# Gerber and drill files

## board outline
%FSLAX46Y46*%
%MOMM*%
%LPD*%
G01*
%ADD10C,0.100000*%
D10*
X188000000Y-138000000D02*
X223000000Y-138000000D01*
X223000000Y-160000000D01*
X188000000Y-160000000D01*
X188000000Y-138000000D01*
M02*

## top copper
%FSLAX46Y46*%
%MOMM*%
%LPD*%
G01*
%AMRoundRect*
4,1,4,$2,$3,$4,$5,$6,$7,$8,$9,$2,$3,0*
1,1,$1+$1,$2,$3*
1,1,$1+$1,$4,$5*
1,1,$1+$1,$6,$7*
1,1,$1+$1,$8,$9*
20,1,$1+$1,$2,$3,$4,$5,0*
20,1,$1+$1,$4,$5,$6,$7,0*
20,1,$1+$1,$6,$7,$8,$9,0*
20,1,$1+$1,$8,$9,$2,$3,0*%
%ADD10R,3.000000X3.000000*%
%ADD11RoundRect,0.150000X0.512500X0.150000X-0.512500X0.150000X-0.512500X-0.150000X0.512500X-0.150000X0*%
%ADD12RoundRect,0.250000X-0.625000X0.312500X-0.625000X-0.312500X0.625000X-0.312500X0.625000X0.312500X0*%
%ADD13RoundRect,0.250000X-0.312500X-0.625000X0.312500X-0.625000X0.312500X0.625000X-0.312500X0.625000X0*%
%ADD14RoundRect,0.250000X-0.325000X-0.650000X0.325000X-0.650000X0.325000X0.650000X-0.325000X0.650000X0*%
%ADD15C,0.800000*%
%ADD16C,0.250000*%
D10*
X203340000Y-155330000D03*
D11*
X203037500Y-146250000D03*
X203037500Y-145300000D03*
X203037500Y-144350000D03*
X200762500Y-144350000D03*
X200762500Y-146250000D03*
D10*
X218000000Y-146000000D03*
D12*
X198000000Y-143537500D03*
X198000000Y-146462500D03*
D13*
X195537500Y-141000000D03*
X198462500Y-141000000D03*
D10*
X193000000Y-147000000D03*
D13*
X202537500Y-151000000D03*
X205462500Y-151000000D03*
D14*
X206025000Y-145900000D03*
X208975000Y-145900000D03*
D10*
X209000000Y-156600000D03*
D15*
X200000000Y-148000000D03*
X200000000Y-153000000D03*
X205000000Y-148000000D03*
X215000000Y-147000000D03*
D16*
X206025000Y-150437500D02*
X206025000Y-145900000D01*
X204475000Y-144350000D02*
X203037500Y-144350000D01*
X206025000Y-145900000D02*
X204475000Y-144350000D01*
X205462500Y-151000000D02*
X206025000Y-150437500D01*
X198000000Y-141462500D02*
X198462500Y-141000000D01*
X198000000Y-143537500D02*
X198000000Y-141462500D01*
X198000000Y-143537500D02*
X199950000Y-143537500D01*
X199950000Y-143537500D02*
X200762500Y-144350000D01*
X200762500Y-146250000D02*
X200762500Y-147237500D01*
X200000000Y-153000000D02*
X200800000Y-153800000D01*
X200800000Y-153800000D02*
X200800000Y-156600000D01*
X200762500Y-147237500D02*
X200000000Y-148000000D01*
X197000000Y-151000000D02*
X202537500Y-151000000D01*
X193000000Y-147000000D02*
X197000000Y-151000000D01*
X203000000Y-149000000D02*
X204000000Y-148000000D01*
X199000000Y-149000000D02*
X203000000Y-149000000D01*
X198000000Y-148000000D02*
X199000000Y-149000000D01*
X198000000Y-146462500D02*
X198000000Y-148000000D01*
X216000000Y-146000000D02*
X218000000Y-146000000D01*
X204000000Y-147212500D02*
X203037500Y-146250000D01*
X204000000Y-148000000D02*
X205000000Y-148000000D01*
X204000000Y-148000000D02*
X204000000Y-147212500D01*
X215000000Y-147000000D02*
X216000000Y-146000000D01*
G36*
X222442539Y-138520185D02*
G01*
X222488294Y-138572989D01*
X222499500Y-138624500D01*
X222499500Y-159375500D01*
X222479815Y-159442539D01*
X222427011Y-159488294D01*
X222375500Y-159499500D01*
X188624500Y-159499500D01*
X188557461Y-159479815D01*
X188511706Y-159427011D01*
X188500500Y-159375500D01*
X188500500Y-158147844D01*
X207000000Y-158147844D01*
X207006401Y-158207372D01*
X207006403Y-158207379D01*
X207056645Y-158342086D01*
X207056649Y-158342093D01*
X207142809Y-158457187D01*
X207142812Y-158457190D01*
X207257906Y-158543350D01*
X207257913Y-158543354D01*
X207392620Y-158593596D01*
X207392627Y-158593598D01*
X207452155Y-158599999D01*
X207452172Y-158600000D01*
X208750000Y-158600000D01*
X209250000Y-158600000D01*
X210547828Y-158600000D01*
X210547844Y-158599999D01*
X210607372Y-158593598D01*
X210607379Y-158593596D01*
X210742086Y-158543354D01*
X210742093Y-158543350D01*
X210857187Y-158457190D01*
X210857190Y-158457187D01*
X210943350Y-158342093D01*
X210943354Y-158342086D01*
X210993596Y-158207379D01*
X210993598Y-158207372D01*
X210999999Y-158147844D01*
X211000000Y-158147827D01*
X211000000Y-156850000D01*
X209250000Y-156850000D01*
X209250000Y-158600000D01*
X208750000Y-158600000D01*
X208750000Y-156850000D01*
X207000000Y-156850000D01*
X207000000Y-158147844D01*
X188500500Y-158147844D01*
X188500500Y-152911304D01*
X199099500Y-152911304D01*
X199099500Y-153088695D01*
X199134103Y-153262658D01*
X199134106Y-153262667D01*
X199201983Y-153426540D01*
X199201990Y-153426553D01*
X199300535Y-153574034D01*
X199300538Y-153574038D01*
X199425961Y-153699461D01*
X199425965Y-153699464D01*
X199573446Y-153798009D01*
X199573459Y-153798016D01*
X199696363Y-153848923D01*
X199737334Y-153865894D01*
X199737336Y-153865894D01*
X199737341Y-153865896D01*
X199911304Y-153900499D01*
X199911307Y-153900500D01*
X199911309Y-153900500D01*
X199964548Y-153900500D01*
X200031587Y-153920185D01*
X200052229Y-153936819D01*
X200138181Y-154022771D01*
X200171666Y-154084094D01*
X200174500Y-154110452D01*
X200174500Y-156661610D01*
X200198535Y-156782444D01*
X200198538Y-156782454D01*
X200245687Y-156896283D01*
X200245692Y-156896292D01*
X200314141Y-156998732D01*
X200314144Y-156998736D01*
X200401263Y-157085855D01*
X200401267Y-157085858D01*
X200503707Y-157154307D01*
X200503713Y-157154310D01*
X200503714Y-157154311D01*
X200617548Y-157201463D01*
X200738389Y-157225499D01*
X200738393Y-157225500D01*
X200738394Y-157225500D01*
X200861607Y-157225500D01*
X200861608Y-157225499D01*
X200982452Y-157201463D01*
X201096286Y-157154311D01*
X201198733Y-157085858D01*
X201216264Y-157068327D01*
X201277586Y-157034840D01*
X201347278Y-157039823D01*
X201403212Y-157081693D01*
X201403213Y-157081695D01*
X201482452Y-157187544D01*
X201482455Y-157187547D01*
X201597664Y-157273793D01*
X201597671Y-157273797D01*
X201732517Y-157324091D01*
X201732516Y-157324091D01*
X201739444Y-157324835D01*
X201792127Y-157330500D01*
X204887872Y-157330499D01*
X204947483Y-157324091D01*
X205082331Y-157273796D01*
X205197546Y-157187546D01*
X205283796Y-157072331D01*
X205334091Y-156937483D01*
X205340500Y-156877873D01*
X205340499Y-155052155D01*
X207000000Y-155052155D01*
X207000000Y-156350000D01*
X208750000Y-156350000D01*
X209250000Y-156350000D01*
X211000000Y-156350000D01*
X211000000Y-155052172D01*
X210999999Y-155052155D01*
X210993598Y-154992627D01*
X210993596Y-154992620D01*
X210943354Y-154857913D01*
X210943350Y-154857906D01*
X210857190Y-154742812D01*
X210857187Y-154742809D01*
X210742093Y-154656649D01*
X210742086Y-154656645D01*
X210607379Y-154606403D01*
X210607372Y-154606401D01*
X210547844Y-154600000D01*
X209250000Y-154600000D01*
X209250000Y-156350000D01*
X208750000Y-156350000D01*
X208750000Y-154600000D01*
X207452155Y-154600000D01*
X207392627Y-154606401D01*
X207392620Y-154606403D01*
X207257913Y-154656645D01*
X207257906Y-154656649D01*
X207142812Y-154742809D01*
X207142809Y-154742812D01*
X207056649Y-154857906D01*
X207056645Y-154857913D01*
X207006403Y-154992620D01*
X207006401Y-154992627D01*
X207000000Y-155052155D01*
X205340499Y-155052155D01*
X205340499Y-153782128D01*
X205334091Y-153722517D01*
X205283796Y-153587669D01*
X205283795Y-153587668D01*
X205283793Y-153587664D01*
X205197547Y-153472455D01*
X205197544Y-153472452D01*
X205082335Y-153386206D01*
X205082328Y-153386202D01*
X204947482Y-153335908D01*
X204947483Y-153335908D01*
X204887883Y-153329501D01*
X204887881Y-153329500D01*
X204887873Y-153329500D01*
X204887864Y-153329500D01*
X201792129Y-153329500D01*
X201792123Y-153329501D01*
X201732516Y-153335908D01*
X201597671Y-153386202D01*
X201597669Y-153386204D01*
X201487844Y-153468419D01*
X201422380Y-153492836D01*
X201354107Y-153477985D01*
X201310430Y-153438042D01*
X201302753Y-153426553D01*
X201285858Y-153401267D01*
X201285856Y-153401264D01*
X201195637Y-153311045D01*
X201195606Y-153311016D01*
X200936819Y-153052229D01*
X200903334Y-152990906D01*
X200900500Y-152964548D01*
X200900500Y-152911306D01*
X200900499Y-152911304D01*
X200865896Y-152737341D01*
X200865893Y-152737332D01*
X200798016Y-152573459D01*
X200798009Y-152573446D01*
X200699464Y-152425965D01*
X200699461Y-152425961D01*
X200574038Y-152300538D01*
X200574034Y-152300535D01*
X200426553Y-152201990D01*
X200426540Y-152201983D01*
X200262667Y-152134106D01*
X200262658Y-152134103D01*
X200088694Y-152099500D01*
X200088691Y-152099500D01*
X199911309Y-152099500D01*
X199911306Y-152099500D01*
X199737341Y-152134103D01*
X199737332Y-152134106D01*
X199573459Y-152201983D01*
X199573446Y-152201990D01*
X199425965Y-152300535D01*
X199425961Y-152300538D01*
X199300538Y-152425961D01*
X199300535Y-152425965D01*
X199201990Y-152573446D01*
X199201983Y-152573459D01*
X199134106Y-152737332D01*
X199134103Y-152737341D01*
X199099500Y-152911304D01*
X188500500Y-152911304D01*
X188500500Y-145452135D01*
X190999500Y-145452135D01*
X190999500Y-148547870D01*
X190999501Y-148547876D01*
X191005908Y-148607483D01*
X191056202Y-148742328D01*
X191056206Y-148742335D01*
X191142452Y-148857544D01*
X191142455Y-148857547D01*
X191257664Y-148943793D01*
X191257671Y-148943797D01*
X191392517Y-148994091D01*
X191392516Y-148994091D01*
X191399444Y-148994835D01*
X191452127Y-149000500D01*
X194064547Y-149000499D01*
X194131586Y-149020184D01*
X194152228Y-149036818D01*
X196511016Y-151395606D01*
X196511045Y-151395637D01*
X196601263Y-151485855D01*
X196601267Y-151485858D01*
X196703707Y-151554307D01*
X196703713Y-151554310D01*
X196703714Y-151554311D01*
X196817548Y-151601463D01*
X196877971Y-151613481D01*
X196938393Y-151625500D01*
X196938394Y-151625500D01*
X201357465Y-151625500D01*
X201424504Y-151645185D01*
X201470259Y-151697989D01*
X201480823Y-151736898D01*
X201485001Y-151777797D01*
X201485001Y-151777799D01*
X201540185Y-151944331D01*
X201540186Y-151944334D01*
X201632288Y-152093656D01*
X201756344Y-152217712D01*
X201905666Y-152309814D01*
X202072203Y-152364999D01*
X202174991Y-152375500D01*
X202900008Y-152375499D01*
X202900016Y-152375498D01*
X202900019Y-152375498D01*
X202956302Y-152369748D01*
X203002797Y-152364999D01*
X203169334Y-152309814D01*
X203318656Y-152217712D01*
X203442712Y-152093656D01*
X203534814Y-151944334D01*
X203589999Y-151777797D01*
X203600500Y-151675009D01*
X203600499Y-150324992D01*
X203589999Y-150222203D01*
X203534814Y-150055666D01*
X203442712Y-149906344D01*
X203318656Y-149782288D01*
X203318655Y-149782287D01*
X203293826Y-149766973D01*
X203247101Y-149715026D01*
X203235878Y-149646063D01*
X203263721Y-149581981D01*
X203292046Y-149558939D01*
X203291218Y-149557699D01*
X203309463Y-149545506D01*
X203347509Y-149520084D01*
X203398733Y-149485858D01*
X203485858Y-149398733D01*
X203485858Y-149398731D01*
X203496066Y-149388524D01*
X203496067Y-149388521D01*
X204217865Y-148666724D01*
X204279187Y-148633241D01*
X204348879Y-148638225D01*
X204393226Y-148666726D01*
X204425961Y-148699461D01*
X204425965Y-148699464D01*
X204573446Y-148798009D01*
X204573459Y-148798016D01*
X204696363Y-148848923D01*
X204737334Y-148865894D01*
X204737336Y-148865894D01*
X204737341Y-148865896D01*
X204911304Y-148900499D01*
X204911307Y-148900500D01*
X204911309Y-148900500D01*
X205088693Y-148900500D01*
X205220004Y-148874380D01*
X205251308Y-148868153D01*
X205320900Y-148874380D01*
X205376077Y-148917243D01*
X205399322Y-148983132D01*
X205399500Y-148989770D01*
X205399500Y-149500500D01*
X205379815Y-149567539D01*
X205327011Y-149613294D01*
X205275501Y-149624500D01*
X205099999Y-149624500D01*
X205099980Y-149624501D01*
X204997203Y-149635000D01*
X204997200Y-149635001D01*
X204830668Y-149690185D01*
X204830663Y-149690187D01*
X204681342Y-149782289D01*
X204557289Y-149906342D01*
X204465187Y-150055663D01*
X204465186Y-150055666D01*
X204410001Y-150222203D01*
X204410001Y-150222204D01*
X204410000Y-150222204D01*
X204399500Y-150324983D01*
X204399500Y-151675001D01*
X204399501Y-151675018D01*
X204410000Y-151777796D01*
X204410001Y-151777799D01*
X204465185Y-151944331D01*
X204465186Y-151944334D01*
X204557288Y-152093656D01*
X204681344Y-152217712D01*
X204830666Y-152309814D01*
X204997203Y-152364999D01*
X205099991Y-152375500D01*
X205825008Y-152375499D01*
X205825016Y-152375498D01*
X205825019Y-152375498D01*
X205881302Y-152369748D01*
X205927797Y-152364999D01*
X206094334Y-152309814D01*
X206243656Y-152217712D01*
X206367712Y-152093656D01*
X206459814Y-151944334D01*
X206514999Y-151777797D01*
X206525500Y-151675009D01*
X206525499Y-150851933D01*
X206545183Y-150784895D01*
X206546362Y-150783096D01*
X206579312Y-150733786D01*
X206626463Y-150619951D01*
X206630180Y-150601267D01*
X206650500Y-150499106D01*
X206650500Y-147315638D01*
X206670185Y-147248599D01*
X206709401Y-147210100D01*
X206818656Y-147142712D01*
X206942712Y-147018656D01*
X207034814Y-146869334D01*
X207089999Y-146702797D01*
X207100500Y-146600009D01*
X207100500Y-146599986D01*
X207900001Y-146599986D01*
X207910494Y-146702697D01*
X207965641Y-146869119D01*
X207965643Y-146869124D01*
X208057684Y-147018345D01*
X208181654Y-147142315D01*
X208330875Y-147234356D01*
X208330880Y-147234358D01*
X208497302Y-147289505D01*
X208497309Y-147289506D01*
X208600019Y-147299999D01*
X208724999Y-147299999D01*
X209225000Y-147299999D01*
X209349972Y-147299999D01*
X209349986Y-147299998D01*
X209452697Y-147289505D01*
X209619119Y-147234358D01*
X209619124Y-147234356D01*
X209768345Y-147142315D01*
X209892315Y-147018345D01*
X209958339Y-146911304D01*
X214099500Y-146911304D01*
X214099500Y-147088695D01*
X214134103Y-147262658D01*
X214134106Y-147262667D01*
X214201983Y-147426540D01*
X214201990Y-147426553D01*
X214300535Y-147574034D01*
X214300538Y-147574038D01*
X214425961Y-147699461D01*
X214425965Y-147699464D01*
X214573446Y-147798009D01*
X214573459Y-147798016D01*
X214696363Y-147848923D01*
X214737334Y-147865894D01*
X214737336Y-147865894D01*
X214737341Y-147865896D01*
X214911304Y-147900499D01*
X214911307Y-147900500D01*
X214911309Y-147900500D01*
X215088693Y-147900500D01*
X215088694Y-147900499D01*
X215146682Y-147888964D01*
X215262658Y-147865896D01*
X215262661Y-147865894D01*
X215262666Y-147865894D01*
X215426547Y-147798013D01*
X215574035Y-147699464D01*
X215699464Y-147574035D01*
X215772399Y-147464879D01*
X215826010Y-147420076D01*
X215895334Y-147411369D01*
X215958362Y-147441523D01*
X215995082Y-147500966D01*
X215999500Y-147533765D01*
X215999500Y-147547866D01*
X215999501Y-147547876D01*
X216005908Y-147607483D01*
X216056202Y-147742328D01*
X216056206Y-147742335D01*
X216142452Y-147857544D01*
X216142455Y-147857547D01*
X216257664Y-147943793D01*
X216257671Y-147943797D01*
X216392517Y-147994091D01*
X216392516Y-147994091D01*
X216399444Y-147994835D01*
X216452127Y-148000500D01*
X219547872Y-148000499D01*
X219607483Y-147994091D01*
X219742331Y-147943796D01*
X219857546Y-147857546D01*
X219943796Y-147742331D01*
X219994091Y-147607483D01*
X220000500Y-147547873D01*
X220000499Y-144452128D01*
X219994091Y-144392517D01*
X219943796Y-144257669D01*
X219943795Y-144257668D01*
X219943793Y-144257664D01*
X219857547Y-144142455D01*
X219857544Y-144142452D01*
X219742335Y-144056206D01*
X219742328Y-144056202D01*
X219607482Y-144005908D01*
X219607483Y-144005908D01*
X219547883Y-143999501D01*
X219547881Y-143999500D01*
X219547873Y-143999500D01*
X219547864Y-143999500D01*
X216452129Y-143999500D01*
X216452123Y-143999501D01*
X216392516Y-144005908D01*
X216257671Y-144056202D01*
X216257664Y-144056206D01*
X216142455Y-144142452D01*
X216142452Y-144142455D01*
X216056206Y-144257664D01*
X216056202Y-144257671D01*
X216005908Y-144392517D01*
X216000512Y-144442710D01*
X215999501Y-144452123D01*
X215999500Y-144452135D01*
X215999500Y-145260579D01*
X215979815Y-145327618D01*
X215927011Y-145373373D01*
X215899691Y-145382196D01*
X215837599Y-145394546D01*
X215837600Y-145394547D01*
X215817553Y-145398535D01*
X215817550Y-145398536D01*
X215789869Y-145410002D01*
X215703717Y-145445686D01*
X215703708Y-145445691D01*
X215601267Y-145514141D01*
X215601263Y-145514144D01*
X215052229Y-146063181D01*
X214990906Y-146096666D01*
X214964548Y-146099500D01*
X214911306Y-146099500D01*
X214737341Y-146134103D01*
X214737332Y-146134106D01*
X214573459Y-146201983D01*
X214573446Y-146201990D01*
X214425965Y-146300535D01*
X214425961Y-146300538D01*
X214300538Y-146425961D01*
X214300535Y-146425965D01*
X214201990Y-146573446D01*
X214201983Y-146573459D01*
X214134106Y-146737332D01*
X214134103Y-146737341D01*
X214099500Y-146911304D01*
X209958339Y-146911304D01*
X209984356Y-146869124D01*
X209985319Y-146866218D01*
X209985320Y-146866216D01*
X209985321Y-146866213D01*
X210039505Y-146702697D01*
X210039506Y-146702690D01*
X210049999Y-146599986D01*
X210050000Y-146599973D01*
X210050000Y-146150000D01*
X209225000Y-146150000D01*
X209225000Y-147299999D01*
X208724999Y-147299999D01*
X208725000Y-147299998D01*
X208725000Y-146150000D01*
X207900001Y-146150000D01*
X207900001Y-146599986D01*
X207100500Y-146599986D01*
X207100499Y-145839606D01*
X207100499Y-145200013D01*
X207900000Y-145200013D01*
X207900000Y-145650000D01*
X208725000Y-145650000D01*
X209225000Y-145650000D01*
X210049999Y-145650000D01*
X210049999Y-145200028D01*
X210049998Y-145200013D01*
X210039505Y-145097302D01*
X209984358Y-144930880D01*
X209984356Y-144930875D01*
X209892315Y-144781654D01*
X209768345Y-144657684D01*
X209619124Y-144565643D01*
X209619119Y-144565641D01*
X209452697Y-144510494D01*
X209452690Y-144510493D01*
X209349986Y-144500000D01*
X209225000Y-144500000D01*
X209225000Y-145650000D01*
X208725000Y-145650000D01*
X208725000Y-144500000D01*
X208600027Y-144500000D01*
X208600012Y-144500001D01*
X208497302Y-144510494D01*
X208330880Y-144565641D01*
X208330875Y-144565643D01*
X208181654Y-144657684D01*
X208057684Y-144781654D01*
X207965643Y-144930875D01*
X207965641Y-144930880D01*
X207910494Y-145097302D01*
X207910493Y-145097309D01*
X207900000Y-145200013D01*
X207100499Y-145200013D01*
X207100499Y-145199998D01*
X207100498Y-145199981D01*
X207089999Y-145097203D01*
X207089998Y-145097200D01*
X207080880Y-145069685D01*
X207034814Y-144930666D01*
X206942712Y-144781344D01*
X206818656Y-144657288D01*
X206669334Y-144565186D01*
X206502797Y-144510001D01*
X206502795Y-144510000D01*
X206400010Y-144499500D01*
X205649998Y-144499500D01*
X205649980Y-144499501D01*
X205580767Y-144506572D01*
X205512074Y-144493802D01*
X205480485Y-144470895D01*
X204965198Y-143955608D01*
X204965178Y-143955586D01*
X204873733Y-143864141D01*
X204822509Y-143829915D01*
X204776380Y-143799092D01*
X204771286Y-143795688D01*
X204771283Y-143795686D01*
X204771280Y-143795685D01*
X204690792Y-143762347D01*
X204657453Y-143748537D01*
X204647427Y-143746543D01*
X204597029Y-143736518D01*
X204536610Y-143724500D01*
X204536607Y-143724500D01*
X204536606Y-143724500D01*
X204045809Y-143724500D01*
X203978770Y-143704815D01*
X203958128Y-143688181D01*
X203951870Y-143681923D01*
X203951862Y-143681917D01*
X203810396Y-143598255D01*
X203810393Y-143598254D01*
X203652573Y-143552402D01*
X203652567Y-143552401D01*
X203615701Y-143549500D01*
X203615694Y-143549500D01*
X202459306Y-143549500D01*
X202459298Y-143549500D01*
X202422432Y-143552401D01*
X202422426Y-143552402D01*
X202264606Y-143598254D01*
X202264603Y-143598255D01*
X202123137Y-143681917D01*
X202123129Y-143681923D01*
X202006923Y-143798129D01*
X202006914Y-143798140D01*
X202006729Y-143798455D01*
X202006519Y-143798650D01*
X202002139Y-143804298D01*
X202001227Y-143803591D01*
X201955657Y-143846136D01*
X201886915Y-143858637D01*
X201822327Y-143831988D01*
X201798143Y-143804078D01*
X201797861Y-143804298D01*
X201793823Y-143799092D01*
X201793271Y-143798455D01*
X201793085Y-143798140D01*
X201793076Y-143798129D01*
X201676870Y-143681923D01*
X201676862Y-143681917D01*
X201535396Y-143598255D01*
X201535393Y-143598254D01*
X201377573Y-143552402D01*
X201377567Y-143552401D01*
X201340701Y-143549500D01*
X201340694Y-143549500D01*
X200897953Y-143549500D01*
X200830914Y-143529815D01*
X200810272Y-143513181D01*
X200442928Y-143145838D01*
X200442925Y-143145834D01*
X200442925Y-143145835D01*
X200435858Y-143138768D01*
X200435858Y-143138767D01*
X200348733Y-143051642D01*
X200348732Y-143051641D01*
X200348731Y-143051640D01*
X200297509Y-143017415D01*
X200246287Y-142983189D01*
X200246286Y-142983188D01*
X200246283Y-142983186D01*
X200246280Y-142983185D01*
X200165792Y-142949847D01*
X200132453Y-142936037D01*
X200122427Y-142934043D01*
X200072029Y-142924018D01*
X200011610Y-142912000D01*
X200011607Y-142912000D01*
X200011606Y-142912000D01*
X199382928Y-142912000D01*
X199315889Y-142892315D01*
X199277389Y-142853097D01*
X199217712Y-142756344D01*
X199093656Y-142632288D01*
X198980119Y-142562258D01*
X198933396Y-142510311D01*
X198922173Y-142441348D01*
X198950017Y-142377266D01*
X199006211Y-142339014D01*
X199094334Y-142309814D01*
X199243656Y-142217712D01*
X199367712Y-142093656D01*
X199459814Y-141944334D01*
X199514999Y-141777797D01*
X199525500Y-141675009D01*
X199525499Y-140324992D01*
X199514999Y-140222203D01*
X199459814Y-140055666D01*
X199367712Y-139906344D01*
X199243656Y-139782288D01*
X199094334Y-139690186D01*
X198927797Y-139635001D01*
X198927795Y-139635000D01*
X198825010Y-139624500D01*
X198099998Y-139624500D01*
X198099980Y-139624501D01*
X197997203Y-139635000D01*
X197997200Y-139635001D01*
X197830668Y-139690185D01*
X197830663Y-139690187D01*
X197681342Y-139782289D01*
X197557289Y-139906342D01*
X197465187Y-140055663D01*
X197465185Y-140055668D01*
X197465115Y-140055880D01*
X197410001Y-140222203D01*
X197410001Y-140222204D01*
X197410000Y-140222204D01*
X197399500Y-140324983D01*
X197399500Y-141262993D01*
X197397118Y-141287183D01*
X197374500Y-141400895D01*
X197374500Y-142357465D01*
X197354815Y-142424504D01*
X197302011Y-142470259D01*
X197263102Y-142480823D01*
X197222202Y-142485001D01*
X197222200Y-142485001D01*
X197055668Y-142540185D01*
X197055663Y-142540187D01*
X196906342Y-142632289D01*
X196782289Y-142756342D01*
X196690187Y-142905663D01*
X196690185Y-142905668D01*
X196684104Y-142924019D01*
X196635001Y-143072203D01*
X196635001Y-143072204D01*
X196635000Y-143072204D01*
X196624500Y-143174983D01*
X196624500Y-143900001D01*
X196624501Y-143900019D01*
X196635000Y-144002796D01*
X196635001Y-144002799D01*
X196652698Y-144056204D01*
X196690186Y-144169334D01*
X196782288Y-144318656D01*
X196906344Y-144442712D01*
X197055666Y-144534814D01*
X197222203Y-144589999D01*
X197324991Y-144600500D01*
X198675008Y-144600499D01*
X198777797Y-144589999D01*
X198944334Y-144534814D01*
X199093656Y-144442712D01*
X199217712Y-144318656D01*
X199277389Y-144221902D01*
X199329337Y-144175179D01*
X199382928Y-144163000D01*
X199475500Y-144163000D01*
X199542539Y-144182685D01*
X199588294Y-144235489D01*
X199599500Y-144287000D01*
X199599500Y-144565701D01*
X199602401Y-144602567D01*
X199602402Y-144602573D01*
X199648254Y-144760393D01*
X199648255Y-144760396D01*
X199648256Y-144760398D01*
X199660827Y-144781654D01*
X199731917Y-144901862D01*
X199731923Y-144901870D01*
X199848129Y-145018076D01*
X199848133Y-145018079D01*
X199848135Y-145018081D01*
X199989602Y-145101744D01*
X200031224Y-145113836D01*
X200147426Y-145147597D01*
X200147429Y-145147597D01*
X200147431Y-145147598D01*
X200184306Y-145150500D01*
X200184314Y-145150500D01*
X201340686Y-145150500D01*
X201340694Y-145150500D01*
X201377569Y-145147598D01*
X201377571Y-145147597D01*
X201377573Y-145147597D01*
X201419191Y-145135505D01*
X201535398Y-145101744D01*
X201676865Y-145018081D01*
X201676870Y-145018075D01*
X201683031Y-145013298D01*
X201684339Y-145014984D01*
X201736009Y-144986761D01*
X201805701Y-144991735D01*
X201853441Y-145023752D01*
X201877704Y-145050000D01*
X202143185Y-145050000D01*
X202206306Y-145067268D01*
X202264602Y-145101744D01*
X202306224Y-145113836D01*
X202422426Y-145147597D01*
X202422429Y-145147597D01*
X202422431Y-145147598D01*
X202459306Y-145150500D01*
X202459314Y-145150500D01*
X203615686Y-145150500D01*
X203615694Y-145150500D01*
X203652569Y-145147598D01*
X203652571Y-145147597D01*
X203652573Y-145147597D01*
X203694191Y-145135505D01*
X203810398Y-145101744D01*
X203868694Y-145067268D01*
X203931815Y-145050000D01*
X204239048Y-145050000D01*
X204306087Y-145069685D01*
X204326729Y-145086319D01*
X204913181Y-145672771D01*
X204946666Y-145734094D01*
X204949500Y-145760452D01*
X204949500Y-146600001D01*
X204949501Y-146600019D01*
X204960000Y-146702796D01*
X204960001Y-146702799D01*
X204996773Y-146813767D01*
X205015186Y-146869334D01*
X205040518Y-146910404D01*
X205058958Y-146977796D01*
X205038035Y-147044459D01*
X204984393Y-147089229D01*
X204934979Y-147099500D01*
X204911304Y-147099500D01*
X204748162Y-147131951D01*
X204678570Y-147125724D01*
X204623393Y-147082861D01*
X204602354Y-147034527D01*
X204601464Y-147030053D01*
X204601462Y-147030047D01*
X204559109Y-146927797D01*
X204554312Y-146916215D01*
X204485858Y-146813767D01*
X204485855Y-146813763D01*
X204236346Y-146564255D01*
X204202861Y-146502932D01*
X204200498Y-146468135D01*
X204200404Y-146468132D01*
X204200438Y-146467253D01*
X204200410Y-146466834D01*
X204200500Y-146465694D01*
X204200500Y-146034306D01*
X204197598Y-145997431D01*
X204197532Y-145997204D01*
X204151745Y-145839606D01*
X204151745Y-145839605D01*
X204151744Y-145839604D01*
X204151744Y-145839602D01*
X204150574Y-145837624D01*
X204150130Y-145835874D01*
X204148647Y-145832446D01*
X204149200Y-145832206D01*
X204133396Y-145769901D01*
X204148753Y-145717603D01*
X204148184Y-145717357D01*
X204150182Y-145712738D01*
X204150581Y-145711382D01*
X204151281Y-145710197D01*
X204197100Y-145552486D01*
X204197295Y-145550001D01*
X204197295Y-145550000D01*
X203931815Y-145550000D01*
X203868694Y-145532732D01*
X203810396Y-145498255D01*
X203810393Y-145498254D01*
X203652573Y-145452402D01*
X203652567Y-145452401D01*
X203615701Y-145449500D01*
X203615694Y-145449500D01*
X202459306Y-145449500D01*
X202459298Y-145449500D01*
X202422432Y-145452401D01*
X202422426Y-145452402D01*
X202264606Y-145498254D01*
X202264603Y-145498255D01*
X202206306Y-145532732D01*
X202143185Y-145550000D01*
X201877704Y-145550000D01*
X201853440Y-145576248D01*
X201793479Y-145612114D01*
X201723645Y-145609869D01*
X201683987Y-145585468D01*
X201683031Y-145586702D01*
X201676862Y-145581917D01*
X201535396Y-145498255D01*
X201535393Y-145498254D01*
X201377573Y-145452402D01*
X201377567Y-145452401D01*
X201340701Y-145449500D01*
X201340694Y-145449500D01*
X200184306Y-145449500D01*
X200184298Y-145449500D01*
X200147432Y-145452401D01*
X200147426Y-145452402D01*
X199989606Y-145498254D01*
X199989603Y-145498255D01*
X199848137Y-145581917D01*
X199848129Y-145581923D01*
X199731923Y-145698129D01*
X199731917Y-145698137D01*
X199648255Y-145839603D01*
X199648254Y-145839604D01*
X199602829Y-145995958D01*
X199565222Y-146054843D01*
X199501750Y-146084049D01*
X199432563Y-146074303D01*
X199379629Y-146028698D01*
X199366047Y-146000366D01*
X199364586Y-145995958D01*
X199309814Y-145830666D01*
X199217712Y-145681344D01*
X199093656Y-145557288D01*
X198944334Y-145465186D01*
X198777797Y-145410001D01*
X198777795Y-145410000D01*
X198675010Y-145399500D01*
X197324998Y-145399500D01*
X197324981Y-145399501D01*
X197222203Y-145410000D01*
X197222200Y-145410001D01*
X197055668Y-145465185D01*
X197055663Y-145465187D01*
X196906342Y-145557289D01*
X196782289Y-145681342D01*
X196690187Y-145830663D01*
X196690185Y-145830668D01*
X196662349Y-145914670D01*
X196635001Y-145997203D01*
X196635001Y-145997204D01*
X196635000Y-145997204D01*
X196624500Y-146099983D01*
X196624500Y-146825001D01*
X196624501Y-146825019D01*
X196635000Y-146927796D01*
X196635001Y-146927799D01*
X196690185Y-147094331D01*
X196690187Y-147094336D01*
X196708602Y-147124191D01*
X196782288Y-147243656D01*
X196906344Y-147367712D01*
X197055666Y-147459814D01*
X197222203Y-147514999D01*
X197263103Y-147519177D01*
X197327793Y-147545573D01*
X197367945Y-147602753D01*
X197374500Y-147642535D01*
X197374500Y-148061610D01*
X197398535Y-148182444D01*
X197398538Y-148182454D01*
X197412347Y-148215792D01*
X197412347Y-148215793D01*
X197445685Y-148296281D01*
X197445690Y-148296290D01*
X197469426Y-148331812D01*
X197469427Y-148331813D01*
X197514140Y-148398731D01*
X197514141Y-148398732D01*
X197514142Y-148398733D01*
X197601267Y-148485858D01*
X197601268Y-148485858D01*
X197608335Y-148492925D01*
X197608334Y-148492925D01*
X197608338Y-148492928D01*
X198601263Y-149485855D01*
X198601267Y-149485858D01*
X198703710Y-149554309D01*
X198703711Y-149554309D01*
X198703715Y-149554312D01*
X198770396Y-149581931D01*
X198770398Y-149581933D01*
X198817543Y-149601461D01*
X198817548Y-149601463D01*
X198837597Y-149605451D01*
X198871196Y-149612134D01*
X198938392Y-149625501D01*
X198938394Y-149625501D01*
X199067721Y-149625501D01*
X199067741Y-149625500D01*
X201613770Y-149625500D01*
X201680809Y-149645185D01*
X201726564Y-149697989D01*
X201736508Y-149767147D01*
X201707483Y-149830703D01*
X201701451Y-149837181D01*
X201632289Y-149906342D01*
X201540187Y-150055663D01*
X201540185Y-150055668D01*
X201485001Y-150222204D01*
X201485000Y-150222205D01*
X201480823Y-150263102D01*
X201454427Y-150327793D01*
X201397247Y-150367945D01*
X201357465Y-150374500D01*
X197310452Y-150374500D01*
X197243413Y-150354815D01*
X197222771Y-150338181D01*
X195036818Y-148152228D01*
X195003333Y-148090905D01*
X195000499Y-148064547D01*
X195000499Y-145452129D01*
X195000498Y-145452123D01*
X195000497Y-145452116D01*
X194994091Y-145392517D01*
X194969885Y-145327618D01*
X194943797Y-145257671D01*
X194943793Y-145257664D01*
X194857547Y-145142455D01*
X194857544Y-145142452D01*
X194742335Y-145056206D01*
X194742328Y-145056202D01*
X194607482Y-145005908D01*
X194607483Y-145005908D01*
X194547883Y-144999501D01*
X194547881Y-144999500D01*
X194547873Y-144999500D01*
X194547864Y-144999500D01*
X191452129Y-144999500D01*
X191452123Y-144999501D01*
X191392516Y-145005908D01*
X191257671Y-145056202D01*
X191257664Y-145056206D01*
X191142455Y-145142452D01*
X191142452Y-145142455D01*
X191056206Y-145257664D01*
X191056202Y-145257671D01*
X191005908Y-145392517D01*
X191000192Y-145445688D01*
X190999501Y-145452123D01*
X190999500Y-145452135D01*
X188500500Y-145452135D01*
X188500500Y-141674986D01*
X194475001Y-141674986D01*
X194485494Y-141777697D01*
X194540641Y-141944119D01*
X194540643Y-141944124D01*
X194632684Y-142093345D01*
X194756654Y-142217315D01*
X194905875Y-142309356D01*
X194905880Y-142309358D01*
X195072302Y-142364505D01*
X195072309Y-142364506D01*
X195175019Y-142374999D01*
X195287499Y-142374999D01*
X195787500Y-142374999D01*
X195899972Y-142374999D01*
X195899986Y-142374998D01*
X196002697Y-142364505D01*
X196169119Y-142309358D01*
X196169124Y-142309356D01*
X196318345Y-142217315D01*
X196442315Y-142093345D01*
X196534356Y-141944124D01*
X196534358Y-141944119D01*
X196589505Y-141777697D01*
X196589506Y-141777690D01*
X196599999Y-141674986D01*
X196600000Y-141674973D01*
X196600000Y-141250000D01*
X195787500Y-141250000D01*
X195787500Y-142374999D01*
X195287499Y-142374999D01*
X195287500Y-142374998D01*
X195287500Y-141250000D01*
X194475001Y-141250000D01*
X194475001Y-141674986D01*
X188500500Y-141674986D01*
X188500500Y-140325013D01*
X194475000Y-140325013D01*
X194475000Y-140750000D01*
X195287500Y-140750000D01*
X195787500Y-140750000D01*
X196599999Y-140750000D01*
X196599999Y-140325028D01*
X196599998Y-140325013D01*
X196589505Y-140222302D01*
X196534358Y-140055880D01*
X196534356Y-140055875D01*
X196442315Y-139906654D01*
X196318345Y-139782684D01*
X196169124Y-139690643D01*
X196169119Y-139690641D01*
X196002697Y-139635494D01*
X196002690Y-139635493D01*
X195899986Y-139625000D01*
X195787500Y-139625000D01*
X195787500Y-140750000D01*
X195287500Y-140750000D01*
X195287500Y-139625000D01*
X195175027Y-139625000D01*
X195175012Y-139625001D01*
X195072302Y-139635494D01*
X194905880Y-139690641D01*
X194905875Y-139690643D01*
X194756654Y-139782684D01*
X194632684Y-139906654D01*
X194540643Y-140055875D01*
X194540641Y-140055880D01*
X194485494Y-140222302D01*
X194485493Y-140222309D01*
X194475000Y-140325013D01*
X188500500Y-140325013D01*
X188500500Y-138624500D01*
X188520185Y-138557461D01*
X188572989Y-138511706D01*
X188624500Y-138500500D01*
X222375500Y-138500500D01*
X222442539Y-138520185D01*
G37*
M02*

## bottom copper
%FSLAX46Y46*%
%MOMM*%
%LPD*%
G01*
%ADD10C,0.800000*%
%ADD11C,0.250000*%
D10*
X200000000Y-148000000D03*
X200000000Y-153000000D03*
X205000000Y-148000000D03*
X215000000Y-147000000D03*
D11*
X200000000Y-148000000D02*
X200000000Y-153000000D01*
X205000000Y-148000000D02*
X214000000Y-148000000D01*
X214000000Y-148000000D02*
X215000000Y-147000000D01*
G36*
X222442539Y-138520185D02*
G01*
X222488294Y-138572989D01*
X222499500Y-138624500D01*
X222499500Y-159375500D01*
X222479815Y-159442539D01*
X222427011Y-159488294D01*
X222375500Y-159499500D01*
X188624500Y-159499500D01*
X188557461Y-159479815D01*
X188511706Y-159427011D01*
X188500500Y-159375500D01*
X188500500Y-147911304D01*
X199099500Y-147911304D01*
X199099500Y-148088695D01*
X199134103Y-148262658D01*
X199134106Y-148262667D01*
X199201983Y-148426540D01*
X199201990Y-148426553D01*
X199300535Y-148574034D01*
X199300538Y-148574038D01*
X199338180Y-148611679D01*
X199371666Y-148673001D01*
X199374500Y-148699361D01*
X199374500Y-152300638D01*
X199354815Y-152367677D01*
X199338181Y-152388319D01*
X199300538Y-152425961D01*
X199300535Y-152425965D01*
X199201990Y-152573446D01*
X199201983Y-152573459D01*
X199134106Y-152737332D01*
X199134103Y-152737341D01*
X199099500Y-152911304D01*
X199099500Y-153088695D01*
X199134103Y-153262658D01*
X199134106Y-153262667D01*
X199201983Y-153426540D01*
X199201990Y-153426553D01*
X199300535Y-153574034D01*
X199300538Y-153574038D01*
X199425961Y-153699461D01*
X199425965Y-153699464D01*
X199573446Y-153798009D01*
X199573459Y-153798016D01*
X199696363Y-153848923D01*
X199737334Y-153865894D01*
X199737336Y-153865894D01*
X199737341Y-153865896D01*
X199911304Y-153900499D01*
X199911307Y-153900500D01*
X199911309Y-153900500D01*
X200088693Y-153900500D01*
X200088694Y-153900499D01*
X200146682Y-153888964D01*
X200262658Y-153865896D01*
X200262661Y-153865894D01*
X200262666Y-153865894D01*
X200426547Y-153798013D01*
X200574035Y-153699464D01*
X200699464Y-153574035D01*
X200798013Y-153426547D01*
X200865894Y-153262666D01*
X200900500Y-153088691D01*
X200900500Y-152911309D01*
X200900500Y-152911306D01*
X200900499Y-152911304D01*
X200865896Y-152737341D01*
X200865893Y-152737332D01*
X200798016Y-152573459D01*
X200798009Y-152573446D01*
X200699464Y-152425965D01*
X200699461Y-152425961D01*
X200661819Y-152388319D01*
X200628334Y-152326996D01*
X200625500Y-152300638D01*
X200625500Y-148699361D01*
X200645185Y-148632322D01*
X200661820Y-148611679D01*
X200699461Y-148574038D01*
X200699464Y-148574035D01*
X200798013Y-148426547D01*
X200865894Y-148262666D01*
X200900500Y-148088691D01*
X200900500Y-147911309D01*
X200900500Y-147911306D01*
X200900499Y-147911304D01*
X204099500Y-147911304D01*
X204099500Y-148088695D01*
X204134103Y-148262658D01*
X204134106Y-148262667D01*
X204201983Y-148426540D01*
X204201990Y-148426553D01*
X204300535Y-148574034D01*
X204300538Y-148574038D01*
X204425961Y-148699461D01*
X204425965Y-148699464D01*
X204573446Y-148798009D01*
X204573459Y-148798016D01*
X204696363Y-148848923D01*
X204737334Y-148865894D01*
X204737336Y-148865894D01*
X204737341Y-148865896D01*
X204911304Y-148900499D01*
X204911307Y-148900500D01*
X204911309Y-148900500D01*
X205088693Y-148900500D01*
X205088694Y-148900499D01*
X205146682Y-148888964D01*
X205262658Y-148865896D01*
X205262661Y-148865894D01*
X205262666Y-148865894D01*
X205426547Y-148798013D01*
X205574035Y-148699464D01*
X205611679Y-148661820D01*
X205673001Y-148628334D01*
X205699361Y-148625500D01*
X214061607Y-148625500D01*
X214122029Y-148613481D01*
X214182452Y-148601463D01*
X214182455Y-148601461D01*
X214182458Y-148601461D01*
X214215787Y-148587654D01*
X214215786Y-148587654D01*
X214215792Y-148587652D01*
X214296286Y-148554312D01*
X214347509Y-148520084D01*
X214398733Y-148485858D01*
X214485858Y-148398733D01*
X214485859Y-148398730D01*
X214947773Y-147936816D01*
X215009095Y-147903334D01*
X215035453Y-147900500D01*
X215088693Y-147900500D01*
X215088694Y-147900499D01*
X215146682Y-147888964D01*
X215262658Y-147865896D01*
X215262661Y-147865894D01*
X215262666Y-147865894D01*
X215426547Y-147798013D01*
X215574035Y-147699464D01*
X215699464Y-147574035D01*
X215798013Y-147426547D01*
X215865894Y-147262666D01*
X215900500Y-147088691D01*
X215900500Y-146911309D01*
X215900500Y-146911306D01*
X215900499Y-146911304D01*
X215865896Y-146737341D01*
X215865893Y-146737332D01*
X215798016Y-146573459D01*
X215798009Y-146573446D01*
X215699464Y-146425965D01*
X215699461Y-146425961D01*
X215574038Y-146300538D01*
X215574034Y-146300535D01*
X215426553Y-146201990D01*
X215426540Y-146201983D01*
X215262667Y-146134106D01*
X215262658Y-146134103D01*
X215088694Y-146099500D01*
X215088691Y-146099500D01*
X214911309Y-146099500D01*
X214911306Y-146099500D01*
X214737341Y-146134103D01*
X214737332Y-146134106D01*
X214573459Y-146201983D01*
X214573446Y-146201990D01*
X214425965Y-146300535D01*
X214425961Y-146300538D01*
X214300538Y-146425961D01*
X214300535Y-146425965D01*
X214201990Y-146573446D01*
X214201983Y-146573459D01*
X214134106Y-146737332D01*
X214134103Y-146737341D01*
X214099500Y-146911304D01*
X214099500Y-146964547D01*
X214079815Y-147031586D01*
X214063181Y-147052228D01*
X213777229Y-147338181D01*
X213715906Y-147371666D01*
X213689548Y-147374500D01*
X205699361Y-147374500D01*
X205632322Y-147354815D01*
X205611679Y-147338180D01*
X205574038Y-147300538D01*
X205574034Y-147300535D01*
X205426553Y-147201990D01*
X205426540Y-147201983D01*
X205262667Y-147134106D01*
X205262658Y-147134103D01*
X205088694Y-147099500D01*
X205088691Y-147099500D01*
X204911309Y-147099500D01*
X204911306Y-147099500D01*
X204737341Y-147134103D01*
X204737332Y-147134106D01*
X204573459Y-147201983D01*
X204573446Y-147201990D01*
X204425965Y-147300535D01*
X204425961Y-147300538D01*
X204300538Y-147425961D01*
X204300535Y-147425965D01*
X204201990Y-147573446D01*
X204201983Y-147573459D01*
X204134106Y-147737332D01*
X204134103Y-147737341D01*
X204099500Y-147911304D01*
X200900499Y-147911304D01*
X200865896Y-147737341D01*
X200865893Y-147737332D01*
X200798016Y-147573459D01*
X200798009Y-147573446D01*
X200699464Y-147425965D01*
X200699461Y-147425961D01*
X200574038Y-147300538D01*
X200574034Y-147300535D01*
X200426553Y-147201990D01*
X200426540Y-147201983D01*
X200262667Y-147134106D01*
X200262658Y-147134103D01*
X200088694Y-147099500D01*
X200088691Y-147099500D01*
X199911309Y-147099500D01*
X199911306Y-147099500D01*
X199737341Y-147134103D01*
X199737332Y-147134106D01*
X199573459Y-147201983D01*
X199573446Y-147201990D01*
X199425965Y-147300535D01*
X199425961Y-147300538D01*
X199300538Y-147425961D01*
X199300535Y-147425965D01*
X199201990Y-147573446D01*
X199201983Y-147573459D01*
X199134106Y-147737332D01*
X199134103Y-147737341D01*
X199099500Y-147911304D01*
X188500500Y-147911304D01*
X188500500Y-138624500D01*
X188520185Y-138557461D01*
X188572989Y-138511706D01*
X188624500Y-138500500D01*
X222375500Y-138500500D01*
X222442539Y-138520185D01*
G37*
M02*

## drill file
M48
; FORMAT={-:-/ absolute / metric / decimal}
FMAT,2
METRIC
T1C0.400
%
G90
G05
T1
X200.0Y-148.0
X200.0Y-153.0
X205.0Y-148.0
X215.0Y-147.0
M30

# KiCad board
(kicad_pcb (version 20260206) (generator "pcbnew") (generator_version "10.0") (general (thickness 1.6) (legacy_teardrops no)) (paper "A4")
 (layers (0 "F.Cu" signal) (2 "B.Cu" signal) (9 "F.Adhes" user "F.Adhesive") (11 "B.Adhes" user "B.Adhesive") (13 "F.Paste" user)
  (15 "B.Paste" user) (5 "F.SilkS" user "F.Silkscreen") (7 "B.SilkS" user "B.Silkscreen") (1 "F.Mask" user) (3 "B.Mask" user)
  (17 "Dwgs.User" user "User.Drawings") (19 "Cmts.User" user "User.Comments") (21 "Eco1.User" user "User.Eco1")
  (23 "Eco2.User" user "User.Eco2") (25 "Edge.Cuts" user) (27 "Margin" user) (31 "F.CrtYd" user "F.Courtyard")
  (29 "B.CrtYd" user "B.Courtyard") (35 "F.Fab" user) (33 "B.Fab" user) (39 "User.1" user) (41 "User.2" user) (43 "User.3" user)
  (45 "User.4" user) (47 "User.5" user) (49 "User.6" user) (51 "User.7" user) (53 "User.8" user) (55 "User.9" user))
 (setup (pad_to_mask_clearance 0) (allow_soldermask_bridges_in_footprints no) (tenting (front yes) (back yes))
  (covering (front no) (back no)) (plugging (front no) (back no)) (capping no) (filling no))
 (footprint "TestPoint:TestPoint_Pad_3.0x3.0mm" (layer "F.Cu") (at 203.34 155.33)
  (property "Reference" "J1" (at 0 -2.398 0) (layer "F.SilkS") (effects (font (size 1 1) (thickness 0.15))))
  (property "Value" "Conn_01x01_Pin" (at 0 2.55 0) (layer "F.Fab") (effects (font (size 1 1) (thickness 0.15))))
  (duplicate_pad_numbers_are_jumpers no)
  (pad "1" smd rect (at 0 0) (size 3 3) (layers "F.Cu" "F.Mask") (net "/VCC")))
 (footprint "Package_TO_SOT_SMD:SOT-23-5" (layer "F.Cu") (at 201.9 145.3 180)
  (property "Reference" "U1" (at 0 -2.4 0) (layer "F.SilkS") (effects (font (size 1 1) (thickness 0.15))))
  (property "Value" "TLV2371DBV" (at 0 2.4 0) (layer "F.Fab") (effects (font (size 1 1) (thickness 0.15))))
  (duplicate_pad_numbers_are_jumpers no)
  (pad "1" smd roundrect (at -1.1375 -0.95 180) (size 1.325 0.6) (layers "F.Cu" "F.Mask" "F.Paste") (roundrect_rratio 0.25) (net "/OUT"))
  (pad "2" smd roundrect (at -1.1375 0 180) (size 1.325 0.6) (layers "F.Cu" "F.Mask" "F.Paste") (roundrect_rratio 0.25) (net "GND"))
  (pad "3" smd roundrect (at -1.1375 0.95 180) (size 1.325 0.6) (layers "F.Cu" "F.Mask" "F.Paste") (roundrect_rratio 0.25)
   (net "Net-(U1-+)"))
  (pad "4" smd roundrect (at 1.1375 0.95 180) (size 1.325 0.6) (layers "F.Cu" "F.Mask" "F.Paste") (roundrect_rratio 0.25) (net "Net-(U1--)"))
  (pad "5" smd roundrect (at 1.1375 -0.95 180) (size 1.325 0.6) (layers "F.Cu" "F.Mask" "F.Paste") (roundrect_rratio 0.25) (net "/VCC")))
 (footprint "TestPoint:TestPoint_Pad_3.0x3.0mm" (layer "F.Cu") (at 218 146)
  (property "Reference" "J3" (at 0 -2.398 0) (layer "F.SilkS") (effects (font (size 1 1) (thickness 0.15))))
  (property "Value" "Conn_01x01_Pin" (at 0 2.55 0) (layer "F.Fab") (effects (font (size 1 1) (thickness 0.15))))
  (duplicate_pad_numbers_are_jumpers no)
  (pad "1" smd rect (at 0 0) (size 3 3) (layers "F.Cu" "F.Mask") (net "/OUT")))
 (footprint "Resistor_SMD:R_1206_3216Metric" (layer "F.Cu") (at 198 145 -90)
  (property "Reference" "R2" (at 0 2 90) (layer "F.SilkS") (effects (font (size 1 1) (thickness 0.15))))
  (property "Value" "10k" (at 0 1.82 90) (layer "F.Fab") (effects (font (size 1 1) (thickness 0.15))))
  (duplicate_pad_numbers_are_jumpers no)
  (pad "1" smd roundrect (at -1.4625 0 270) (size 1.125 1.75) (layers "F.Cu" "F.Mask" "F.Paste") (roundrect_rratio 0.222222)
   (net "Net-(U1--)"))
  (pad "2" smd roundrect (at 1.4625 0 270) (size 1.125 1.75) (layers "F.Cu" "F.Mask" "F.Paste") (roundrect_rratio 0.222222) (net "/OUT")))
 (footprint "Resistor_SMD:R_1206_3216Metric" (layer "F.Cu") (at 197 141)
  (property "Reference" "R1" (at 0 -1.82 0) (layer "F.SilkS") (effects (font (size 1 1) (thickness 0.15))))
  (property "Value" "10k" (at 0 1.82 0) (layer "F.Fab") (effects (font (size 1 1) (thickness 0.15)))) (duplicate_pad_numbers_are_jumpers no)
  (pad "1" smd roundrect (at -1.4625 0) (size 1.125 1.75) (layers "F.Cu" "F.Mask" "F.Paste") (roundrect_rratio 0.222222) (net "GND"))
  (pad "2" smd roundrect (at 1.4625 0) (size 1.125 1.75) (layers "F.Cu" "F.Mask" "F.Paste") (roundrect_rratio 0.222222) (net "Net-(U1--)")))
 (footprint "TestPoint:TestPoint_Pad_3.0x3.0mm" (layer "F.Cu") (at 193 147)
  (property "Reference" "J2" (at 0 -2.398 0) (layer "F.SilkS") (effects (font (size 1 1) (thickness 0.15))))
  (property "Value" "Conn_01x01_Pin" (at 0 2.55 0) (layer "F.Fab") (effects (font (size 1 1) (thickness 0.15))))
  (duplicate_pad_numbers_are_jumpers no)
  (pad "1" smd rect (at 0 0) (size 3 3) (layers "F.Cu" "F.Mask") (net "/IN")))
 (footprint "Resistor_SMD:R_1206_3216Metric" (layer "F.Cu") (at 204 151)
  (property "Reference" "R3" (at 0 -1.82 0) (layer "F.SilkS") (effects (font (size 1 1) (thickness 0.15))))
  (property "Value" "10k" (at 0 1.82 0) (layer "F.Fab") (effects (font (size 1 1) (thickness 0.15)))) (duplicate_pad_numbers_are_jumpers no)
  (pad "1" smd roundrect (at -1.4625 0) (size 1.125 1.75) (layers "F.Cu" "F.Mask" "F.Paste") (roundrect_rratio 0.222222) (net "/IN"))
  (pad "2" smd roundrect (at 1.4625 0) (size 1.125 1.75) (layers "F.Cu" "F.Mask" "F.Paste") (roundrect_rratio 0.222222) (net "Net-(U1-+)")))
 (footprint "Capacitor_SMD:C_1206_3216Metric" (layer "F.Cu") (at 207.5 145.9)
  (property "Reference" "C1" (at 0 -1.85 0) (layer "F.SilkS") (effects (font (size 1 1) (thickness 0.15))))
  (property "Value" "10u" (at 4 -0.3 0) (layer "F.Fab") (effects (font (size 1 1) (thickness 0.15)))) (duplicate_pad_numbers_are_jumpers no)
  (pad "1" smd roundrect (at -1.475 0) (size 1.15 1.8) (layers "F.Cu" "F.Mask" "F.Paste") (roundrect_rratio 0.217391) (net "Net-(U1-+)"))
  (pad "2" smd roundrect (at 1.475 0) (size 1.15 1.8) (layers "F.Cu" "F.Mask" "F.Paste") (roundrect_rratio 0.217391) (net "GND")))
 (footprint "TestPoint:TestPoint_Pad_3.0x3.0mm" (layer "F.Cu") (at 209 156.6)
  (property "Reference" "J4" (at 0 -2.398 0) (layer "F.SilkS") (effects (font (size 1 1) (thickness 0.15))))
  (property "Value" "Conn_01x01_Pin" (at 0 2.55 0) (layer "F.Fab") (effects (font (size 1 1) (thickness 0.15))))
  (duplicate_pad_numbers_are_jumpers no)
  (pad "1" smd rect (at 0 0) (size 3 3) (layers "F.Cu" "F.Mask") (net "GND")))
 (gr_rect (start 188 138) (end 223 160) (stroke (width 0.1) (type default)) (fill no) (layer "Edge.Cuts"))
 (segment (start 206.025 150.4375) (end 206.025 145.9) (width 0.25) (layer "F.Cu") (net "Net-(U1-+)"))
 (segment (start 204.475 144.35) (end 203.0375 144.35) (width 0.25) (layer "F.Cu") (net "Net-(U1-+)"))
 (segment (start 206.025 145.9) (end 204.475 144.35) (width 0.25) (layer "F.Cu") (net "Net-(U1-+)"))
 (segment (start 205.4625 151) (end 206.025 150.4375) (width 0.25) (layer "F.Cu") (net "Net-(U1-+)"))
 (segment (start 198 141.4625) (end 198.4625 141) (width 0.25) (layer "F.Cu") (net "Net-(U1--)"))
 (segment (start 198 143.5375) (end 198 141.4625) (width 0.25) (layer "F.Cu") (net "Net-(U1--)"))
 (segment (start 198 143.5375) (end 199.95 143.5375) (width 0.25) (layer "F.Cu") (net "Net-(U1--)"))
 (segment (start 199.95 143.5375) (end 200.7625 144.35) (width 0.25) (layer "F.Cu") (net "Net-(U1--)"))
 (segment (start 200.7625 146.25) (end 200.7625 147.2375) (width 0.25) (layer "F.Cu") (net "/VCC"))
 (segment (start 200 153) (end 200.8 153.8) (width 0.25) (layer "F.Cu") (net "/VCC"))
 (segment (start 200.8 153.8) (end 200.8 156.6) (width 0.25) (layer "F.Cu") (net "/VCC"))
 (segment (start 200.7625 147.2375) (end 200 148) (width 0.25) (layer "F.Cu") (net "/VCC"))
 (via (at 200 148) (size 0.8) (drill 0.4) (layers "F.Cu" "B.Cu") (capping no) (covering (front no) (back no))
  (plugging (front no) (back no)) (filling no) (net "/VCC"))
 (via (at 200 153) (size 0.8) (drill 0.4) (layers "F.Cu" "B.Cu") (capping no) (covering (front no) (back no))
  (plugging (front no) (back no)) (filling no) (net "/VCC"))
 (segment (start 200 148) (end 200 153) (width 0.25) (layer "B.Cu") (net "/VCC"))
 (segment (start 197 151) (end 202.5375 151) (width 0.25) (layer "F.Cu") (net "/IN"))
 (segment (start 193 147) (end 197 151) (width 0.25) (layer "F.Cu") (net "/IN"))
 (segment (start 203 149) (end 204 148) (width 0.25) (layer "F.Cu") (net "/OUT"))
 (segment (start 199 149) (end 203 149) (width 0.25) (layer "F.Cu") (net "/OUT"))
 (segment (start 198 148) (end 199 149) (width 0.25) (layer "F.Cu") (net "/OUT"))
 (segment (start 198 146.4625) (end 198 148) (width 0.25) (layer "F.Cu") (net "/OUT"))
 (segment (start 216 146) (end 218 146) (width 0.25) (layer "F.Cu") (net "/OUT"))
 (segment (start 204 147.2125) (end 203.0375 146.25) (width 0.25) (layer "F.Cu") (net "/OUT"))
 (segment (start 204 148) (end 205 148) (width 0.25) (layer "F.Cu") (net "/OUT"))
 (segment (start 204 148) (end 204 147.2125) (width 0.25) (layer "F.Cu") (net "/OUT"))
 (segment (start 215 147) (end 216 146) (width 0.25) (layer "F.Cu") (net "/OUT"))
 (via (at 205 148) (size 0.8) (drill 0.4) (layers "F.Cu" "B.Cu") (capping no) (covering (front no) (back no))
  (plugging (front no) (back no)) (filling no) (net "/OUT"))
 (via (at 215 147) (size 0.8) (drill 0.4) (layers "F.Cu" "B.Cu") (capping no) (covering (front no) (back no))
  (plugging (front no) (back no)) (filling no) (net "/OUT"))
 (segment (start 205 148) (end 214 148) (width 0.25) (layer "B.Cu") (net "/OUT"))
 (segment (start 214 148) (end 215 147) (width 0.25) (layer "B.Cu") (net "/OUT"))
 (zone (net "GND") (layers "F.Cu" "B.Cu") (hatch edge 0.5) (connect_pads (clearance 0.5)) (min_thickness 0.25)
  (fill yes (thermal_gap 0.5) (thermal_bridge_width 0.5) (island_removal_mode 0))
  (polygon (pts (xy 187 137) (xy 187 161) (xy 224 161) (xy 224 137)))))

